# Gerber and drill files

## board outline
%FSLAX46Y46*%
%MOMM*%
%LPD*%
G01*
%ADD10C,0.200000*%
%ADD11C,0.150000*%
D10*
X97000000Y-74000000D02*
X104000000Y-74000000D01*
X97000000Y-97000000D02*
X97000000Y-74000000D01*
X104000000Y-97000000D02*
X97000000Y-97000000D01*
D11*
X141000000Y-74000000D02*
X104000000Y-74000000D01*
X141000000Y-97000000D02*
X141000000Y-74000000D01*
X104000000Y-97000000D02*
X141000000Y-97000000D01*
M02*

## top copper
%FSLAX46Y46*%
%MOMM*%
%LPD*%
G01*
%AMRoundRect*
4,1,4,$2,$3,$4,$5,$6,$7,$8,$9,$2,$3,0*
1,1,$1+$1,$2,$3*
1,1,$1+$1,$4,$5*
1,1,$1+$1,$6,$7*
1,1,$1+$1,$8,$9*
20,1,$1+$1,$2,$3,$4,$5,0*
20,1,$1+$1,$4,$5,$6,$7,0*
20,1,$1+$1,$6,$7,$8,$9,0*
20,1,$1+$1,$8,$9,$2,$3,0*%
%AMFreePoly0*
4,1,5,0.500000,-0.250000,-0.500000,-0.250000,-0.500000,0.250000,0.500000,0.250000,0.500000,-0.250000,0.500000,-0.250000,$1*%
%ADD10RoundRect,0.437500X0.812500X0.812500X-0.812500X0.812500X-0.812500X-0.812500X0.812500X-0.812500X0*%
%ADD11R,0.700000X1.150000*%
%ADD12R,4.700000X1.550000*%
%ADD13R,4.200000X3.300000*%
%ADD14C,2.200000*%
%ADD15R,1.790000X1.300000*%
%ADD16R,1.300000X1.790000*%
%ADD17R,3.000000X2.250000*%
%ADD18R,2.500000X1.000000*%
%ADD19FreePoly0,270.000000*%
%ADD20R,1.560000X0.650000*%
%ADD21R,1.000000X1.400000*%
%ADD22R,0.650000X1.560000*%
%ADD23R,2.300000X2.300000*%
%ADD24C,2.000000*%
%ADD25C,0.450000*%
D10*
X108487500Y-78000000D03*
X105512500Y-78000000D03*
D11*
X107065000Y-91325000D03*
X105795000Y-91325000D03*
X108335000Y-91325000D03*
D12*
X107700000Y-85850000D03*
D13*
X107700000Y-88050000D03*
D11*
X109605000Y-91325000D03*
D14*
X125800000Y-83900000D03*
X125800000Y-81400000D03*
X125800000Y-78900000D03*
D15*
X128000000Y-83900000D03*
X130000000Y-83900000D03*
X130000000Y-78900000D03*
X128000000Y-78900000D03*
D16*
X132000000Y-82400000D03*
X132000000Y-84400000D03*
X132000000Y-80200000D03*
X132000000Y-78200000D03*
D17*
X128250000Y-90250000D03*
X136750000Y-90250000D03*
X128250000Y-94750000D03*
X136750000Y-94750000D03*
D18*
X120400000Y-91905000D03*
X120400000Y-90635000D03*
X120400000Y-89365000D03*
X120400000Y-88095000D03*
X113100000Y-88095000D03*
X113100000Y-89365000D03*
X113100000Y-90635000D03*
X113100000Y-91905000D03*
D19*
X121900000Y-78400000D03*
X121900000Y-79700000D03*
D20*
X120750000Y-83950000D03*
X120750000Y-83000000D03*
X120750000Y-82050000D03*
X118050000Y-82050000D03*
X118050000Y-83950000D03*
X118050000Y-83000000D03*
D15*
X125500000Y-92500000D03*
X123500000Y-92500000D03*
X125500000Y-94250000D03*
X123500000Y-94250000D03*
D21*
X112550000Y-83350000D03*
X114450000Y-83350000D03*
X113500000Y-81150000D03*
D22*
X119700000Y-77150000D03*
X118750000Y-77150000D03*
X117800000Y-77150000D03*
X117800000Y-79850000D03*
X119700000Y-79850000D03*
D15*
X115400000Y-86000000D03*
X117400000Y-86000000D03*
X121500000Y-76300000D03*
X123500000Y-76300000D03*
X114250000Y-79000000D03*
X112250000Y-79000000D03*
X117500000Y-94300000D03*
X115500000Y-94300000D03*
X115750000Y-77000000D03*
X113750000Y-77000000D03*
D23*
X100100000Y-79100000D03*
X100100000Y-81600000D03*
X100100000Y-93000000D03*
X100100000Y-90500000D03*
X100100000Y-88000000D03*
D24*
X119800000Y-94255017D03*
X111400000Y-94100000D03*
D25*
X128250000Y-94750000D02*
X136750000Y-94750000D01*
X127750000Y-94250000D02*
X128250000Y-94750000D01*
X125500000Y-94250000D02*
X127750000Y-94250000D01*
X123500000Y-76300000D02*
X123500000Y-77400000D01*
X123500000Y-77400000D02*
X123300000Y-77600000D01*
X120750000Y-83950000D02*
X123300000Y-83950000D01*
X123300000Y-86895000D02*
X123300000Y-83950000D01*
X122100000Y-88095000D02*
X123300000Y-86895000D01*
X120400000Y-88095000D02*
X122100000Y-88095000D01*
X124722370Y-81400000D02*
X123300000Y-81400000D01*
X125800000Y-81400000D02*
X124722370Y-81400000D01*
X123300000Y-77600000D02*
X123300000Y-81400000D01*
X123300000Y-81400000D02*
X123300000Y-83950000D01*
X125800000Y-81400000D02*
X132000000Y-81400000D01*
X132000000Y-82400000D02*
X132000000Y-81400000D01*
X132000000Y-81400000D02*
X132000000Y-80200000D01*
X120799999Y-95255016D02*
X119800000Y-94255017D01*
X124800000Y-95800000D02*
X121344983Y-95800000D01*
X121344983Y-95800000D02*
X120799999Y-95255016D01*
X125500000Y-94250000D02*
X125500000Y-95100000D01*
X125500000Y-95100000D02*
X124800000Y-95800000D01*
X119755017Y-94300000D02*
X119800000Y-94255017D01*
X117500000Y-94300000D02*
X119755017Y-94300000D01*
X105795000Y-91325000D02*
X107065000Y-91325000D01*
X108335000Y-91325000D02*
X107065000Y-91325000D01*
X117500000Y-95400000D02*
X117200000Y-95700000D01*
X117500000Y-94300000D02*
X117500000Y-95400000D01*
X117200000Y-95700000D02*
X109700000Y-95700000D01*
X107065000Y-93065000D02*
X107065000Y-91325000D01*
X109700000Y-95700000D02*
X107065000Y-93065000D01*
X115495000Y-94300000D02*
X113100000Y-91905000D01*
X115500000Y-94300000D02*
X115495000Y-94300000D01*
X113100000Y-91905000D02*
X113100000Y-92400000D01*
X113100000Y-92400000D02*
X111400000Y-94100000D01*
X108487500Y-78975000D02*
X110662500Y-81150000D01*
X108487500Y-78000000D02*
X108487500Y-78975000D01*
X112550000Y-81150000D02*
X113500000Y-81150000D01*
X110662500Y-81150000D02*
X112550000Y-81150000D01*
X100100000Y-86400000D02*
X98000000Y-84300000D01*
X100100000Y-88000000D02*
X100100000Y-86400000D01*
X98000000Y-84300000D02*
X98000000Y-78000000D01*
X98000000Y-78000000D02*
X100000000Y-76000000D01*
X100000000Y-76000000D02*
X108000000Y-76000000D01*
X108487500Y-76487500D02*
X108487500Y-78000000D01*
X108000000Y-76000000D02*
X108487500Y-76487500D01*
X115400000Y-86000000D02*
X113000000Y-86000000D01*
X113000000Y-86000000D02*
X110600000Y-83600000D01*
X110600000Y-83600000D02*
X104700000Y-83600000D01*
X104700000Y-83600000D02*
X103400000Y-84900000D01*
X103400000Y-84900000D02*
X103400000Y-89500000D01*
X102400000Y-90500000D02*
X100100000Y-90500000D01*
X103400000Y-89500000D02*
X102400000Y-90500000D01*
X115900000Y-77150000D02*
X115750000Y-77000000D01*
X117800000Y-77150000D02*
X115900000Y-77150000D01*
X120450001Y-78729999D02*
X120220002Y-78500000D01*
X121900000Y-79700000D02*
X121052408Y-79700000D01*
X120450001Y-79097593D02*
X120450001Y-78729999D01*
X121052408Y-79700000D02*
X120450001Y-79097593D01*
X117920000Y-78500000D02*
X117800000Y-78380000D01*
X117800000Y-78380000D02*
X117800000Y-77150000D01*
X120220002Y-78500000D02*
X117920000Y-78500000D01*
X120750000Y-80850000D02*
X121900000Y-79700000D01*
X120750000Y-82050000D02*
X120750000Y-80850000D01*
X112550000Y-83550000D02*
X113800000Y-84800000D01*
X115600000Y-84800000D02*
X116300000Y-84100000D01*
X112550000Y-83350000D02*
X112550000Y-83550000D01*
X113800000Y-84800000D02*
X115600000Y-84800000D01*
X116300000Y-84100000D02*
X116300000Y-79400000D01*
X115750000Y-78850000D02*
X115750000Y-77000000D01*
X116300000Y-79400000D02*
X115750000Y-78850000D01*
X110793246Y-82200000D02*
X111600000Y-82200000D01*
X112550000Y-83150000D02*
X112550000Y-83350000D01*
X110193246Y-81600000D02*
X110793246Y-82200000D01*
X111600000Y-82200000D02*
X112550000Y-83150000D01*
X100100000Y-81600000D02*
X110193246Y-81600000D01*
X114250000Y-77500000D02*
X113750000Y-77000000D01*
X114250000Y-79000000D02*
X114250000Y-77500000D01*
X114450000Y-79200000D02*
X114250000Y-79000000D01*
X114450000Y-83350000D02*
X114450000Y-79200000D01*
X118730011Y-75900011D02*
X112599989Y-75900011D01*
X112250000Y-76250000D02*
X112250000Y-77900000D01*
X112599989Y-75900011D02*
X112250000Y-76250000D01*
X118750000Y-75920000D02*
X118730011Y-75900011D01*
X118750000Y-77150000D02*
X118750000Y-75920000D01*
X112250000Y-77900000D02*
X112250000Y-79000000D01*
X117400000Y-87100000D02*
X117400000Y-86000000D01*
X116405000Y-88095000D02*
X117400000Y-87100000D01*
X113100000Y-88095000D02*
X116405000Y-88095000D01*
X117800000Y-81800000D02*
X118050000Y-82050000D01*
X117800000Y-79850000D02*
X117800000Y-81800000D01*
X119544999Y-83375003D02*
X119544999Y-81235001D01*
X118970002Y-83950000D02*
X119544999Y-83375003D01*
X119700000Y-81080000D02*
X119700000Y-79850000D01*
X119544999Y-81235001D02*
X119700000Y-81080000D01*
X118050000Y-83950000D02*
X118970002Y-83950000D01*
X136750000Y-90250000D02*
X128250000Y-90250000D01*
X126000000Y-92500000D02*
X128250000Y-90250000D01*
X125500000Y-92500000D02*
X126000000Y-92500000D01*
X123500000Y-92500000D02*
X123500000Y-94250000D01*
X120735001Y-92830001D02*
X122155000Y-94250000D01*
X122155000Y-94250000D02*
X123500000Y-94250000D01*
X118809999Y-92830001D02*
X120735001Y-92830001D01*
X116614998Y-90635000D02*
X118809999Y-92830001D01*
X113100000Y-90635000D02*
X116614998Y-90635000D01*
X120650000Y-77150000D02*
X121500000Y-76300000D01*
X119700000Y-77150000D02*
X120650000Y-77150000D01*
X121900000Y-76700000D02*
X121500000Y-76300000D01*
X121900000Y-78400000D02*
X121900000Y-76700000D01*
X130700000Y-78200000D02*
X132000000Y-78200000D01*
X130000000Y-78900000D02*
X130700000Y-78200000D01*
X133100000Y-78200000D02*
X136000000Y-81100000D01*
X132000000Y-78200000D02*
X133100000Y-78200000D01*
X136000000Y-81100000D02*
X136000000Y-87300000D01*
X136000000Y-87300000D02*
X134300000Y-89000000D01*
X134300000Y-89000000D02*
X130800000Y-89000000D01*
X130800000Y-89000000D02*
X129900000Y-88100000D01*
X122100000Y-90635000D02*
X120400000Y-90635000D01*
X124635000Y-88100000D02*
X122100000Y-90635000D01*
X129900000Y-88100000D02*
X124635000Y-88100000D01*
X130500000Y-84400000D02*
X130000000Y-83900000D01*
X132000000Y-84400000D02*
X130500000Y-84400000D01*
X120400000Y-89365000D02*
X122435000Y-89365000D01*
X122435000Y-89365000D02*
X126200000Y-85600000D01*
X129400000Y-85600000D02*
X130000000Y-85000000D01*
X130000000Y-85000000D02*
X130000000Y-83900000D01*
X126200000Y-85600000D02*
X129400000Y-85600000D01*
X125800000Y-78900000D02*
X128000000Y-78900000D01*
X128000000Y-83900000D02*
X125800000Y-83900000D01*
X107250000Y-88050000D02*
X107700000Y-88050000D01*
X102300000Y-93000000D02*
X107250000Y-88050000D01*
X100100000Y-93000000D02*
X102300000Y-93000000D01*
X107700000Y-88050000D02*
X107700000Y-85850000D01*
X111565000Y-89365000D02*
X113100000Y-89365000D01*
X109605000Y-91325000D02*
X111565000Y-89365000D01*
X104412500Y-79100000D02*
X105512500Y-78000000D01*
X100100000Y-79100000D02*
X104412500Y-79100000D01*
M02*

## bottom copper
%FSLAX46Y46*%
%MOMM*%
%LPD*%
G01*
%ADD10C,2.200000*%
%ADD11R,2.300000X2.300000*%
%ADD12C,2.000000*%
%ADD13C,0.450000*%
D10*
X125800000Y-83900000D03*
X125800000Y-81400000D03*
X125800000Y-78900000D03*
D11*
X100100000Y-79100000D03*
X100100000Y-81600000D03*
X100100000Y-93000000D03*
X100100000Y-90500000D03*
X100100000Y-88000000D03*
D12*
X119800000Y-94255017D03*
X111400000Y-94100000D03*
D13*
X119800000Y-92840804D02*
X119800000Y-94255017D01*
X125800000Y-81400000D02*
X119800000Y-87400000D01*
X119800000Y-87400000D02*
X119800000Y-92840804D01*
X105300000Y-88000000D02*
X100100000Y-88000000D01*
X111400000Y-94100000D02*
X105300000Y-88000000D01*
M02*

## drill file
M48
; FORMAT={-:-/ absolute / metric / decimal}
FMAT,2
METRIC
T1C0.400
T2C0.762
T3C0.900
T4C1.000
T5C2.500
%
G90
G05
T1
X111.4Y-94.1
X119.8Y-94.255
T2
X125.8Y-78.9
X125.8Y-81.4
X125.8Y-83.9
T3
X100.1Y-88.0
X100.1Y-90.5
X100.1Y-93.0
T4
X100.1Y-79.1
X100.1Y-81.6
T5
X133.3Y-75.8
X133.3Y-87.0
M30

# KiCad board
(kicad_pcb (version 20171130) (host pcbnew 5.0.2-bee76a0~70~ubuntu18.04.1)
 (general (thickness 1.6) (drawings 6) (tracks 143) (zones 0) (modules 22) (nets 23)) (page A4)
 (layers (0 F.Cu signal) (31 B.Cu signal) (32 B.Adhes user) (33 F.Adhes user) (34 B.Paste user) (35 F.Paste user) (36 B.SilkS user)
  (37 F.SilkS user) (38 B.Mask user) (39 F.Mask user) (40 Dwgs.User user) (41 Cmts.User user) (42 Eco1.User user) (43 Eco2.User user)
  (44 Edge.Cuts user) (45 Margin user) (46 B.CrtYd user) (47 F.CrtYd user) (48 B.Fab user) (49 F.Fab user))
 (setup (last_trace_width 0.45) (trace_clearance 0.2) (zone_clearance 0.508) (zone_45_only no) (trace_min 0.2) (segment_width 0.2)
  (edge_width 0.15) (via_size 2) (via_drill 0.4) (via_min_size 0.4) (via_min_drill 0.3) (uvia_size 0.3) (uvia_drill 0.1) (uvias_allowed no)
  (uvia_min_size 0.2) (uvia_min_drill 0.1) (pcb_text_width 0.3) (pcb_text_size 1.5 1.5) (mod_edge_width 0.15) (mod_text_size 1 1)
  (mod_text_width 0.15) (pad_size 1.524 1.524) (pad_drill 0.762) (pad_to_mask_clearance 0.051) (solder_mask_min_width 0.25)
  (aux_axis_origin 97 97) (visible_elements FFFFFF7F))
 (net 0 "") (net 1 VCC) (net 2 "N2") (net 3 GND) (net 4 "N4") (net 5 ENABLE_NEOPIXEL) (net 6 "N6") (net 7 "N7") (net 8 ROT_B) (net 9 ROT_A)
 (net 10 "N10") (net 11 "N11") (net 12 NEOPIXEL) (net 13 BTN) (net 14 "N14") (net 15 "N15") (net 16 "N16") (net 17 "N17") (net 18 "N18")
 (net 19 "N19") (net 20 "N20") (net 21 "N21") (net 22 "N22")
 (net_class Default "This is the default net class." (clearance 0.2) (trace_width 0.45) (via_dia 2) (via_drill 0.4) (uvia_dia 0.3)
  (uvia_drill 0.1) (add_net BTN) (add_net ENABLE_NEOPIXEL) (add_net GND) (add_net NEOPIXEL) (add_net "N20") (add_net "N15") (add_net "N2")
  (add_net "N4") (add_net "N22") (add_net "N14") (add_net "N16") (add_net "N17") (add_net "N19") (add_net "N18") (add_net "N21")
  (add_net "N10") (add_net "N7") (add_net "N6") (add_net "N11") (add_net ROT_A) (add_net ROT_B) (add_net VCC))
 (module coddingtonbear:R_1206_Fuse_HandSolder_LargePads (layer F.Cu) (at 107 78 180)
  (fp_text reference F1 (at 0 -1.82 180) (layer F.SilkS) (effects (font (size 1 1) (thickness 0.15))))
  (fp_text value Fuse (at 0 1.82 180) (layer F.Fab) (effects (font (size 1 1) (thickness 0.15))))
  (pad 1 smd roundrect (at -1.4875 0 180) (size 2.5 2.5) (layers F.Cu F.Paste F.Mask) (roundrect_rratio 0.175) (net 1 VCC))
  (pad 2 smd roundrect (at 1.4875 0 180) (size 2.5 2.5) (layers F.Cu F.Paste F.Mask) (roundrect_rratio 0.175) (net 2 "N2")))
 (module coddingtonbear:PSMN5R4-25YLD (layer F.Cu) (at 107.7 88.5)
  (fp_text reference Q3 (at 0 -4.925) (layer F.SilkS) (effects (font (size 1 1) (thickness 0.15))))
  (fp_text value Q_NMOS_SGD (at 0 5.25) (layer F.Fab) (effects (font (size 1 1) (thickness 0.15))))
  (pad 7 smd rect (at -1.15 -0.2 90) (size 0.6 0.9) (layers F.Paste))
  (pad 7 smd rect (at -1.15 0.65 90) (size 0.6 0.9) (layers F.Paste))
  (pad 7 smd rect (at -1.15 -1.05 90) (size 0.6 0.9) (layers F.Paste))
  (pad 7 smd rect (at 1.15 -0.2 90) (size 0.6 0.9) (layers F.Paste))
  (pad 7 smd rect (at 1.15 0.65 90) (size 0.6 0.9) (layers F.Paste))
  (pad 7 smd rect (at 1.15 -1.05 90) (size 0.6 0.9) (layers F.Paste))
  (pad 7 smd rect (at 0 -1.05 90) (size 0.6 0.9) (layers F.Paste))
  (pad 7 smd rect (at 0 0.65 90) (size 0.6 0.9) (layers F.Paste))
  (pad 6 smd rect (at -1.875 -2.9) (size 0.6 0.9) (layers F.Paste))
  (pad 6 smd rect (at 1.875 -2.9) (size 0.6 0.9) (layers F.Paste))
  (pad 6 smd rect (at -0.6 -2.9) (size 0.6 0.9) (layers F.Paste))
  (pad 1 smd rect (at -0.635 2.825) (size 0.7 1.15) (layers F.Cu F.Paste F.Mask) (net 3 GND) (solder_mask_margin 0.075)
   (solder_paste_margin -0.05))
  (pad 1 smd rect (at -1.905 2.825) (size 0.7 1.15) (layers F.Cu F.Paste F.Mask) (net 3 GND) (solder_mask_margin 0.075)
   (solder_paste_margin -0.05))
  (pad 1 smd rect (at 0.635 2.825) (size 0.7 1.15) (layers F.Cu F.Paste F.Mask) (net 3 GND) (solder_mask_margin 0.075)
   (solder_paste_margin -0.05))
  (pad 3 smd rect (at 0 -2.65) (size 4.7 1.55) (layers F.Cu F.Mask) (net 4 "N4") (solder_mask_margin 0.075))
  (pad 3 smd rect (at 0 -0.45) (size 4.2 3.3) (layers F.Cu F.Mask) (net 4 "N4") (solder_mask_margin 0.075))
  (pad 2 smd rect (at 1.905 2.825) (size 0.7 1.15) (layers F.Cu F.Paste F.Mask) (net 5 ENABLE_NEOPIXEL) (solder_mask_margin 0.075)
   (solder_paste_margin -0.05))
  (pad 6 smd rect (at 0.6 -2.9) (size 0.6 0.9) (layers F.Paste))
  (pad 7 smd rect (at 0 -0.2 90) (size 0.6 0.9) (layers F.Paste)))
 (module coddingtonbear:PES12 (layer F.Cu) (at 133.3 81.4 270)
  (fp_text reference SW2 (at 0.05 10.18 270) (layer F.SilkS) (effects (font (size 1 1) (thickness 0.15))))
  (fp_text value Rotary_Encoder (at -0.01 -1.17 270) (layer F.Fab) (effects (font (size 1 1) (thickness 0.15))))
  (pad "" np_thru_hole circle (at 5.6 0 270) (size 2.5 2.5) (drill 2.5) (layers *.Cu *.Mask))
  (pad "" np_thru_hole circle (at -5.6 0 270) (size 2.5 2.5) (drill 2.5) (layers *.Cu *.Mask))
  (pad B thru_hole circle (at 2.5 7.5 270) (size 2.2 2.2) (drill 0.762) (layers *.Cu *.Mask) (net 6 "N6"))
  (pad C thru_hole circle (at 0 7.5 270) (size 2.2 2.2) (drill 0.762) (layers *.Cu *.Mask) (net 3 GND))
  (pad A thru_hole circle (at -2.5 7.5 270) (size 2.2 2.2) (drill 0.762) (layers *.Cu *.Mask) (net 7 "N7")))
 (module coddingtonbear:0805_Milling (layer F.Cu) (at 129 83.9)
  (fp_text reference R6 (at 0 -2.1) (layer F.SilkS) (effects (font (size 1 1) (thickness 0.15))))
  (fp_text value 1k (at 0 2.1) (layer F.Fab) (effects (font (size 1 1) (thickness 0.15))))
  (pad 1 smd rect (at -1 0) (size 1.79 1.3) (layers F.Cu F.Paste F.Mask) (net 6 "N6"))
  (pad 2 smd rect (at 1 0) (size 1.79 1.3) (layers F.Cu F.Paste F.Mask) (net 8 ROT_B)))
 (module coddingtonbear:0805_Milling (layer F.Cu) (at 129 78.9)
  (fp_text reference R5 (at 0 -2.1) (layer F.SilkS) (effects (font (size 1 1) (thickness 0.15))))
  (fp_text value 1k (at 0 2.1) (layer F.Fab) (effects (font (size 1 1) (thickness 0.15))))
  (pad 2 smd rect (at 1 0) (size 1.79 1.3) (layers F.Cu F.Paste F.Mask) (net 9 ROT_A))
  (pad 1 smd rect (at -1 0) (size 1.79 1.3) (layers F.Cu F.Paste F.Mask) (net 7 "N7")))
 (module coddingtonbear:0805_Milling (layer F.Cu) (at 132 83.4 270)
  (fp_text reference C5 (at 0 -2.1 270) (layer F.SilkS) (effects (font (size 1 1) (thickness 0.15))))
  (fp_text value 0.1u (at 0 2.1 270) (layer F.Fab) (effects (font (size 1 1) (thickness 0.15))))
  (pad 1 smd rect (at -1 0 270) (size 1.79 1.3) (layers F.Cu F.Paste F.Mask) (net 3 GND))
  (pad 2 smd rect (at 1 0 270) (size 1.79 1.3) (layers F.Cu F.Paste F.Mask) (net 8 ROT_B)))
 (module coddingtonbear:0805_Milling (layer F.Cu) (at 132 79.2 270)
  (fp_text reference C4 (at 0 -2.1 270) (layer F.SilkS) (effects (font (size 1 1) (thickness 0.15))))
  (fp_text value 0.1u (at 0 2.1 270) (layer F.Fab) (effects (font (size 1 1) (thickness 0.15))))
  (pad 2 smd rect (at 1 0 270) (size 1.79 1.3) (layers F.Cu F.Paste F.Mask) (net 3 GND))
  (pad 1 smd rect (at -1 0 270) (size 1.79 1.3) (layers F.Cu F.Paste F.Mask) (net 9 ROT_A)))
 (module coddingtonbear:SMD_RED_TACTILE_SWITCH (layer F.Cu) (at 132.5 92.5)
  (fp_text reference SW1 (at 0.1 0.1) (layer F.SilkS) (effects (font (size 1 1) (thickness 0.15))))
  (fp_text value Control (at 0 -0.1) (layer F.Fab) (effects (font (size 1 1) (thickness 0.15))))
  (pad 1 smd rect (at -4.25 -2.25) (size 3 2.25) (layers F.Cu F.Paste F.Mask) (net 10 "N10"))
  (pad 1 smd rect (at 4.25 -2.25) (size 3 2.25) (layers F.Cu F.Paste F.Mask) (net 10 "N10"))
  (pad 2 smd rect (at -4.25 2.25) (size 3 2.25) (layers F.Cu F.Paste F.Mask) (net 3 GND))
  (pad 2 smd rect (at 4.25 2.25) (size 3 2.25) (layers F.Cu F.Paste F.Mask) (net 3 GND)))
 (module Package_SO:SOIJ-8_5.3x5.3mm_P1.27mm (layer F.Cu) (at 116.75 90 180)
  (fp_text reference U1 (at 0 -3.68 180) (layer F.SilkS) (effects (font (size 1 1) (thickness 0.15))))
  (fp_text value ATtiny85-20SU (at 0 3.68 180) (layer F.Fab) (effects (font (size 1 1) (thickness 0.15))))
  (pad 1 smd rect (at -3.65 -1.905 180) (size 2.5 1) (layers F.Cu F.Paste F.Mask) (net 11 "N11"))
  (pad 2 smd rect (at -3.65 -0.635 180) (size 2.5 1) (layers F.Cu F.Paste F.Mask) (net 9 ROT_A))
  (pad 3 smd rect (at -3.65 0.635 180) (size 2.5 1) (layers F.Cu F.Paste F.Mask) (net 8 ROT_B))
  (pad 4 smd rect (at -3.65 1.905 180) (size 2.5 1) (layers F.Cu F.Paste F.Mask) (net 3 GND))
  (pad 5 smd rect (at 3.65 1.905 180) (size 2.5 1) (layers F.Cu F.Paste F.Mask) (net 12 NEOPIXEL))
  (pad 6 smd rect (at 3.65 0.635 180) (size 2.5 1) (layers F.Cu F.Paste F.Mask) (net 5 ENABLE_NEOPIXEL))
  (pad 7 smd rect (at 3.65 -0.635 180) (size 2.5 1) (layers F.Cu F.Paste F.Mask) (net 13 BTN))
  (pad 8 smd rect (at 3.65 -1.905 180) (size 2.5 1) (layers F.Cu F.Paste F.Mask) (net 1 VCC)))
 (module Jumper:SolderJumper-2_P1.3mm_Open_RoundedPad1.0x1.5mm (layer F.Cu) (at 121.9 79.05 270)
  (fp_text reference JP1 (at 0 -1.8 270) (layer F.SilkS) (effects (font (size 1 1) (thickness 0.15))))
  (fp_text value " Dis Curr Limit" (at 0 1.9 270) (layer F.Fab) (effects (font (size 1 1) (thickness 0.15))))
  (pad 1 smd custom (at -0.65 0 270) (size 1 0.5) (layers F.Cu F.Mask) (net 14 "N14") (zone_connect 0)
   (options (clearance outline) (anchor rect)) (primitives))
  (pad 2 smd custom (at 0.65 0 270) (size 1 0.5) (layers F.Cu F.Mask) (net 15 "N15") (zone_connect 0)
   (options (clearance outline) (anchor rect)) (primitives)))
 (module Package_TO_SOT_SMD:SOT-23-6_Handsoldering (layer F.Cu) (at 119.4 83 180)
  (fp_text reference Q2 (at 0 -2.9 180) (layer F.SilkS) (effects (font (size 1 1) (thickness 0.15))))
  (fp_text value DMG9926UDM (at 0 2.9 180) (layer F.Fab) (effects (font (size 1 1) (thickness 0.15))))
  (pad 1 smd rect (at -1.35 -0.95 180) (size 1.56 0.65) (layers F.Cu F.Paste F.Mask) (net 3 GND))
  (pad 2 smd rect (at -1.35 0 180) (size 1.56 0.65) (layers F.Cu F.Paste F.Mask) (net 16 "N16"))
  (pad 3 smd rect (at -1.35 0.95 180) (size 1.56 0.65) (layers F.Cu F.Paste F.Mask) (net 15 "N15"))
  (pad 4 smd rect (at 1.35 0.95 180) (size 1.56 0.65) (layers F.Cu F.Paste F.Mask) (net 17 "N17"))
  (pad 6 smd rect (at 1.35 -0.95 180) (size 1.56 0.65) (layers F.Cu F.Paste F.Mask) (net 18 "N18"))
  (pad 5 smd rect (at 1.35 0 180) (size 1.56 0.65) (layers F.Cu F.Paste F.Mask) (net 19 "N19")))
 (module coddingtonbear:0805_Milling (layer F.Cu) (at 124.5 92.5 180)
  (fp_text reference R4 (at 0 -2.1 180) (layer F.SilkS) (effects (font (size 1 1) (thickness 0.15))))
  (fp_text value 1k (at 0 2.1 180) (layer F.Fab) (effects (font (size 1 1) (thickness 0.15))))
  (pad 1 smd rect (at -1 0 180) (size 1.79 1.3) (layers F.Cu F.Paste F.Mask) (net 10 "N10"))
  (pad 2 smd rect (at 1 0 180) (size 1.79 1.3) (layers F.Cu F.Paste F.Mask) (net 13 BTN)))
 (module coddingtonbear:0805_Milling (layer F.Cu) (at 124.5 94.25)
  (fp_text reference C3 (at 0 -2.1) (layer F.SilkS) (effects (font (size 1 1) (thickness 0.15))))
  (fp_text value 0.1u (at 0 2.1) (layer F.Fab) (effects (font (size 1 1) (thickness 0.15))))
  (pad 2 smd rect (at 1 0) (size 1.79 1.3) (layers F.Cu F.Paste F.Mask) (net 3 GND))
  (pad 1 smd rect (at -1 0) (size 1.79 1.3) (layers F.Cu F.Paste F.Mask) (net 13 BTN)))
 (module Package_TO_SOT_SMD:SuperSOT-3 (layer F.Cu) (at 113.5 82.25 90)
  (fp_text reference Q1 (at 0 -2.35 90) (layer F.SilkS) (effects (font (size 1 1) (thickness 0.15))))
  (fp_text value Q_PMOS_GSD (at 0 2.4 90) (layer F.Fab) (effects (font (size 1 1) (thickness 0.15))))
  (pad 1 smd rect (at -1.1 -0.95 90) (size 1.4 1) (layers F.Cu F.Paste F.Mask) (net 15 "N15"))
  (pad 2 smd rect (at -1.1 0.95 90) (size 1.4 1) (layers F.Cu F.Paste F.Mask) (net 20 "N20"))
  (pad 3 smd rect (at 1.1 0 90) (size 1.4 1) (layers F.Cu F.Paste F.Mask) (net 1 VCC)))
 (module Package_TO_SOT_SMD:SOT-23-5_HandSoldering (layer F.Cu) (at 118.75 78.5 270)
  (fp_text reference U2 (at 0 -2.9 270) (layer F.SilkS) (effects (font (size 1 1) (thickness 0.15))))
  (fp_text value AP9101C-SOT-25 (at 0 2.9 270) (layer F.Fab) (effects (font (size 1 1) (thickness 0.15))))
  (pad 1 smd rect (at -1.35 -0.95 270) (size 1.56 0.65) (layers F.Cu F.Paste F.Mask) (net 14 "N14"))
  (pad 2 smd rect (at -1.35 0 270) (size 1.56 0.65) (layers F.Cu F.Paste F.Mask) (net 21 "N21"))
  (pad 3 smd rect (at -1.35 0.95 270) (size 1.56 0.65) (layers F.Cu F.Paste F.Mask) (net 15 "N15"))
  (pad 4 smd rect (at 1.35 0.95 270) (size 1.56 0.65) (layers F.Cu F.Paste F.Mask) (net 17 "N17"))
  (pad 5 smd rect (at 1.35 -0.95 270) (size 1.56 0.65) (layers F.Cu F.Paste F.Mask) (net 18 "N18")))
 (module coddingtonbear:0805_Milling (layer F.Cu) (at 116.4 86 180)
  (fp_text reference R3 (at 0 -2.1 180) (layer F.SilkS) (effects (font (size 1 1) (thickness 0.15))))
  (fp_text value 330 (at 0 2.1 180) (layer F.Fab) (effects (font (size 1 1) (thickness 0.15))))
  (pad 2 smd rect (at 1 0 180) (size 1.79 1.3) (layers F.Cu F.Paste F.Mask) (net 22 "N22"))
  (pad 1 smd rect (at -1 0 180) (size 1.79 1.3) (layers F.Cu F.Paste F.Mask) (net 12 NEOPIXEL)))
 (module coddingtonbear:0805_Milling (layer F.Cu) (at 122.5 76.3)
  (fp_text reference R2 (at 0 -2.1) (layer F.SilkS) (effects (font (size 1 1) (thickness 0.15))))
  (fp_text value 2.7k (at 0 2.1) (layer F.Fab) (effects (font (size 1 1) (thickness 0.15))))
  (pad 1 smd rect (at -1 0) (size 1.79 1.3) (layers F.Cu F.Paste F.Mask) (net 14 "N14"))
  (pad 2 smd rect (at 1 0) (size 1.79 1.3) (layers F.Cu F.Paste F.Mask) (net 3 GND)))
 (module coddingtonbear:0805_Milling (layer F.Cu) (at 113.25 79)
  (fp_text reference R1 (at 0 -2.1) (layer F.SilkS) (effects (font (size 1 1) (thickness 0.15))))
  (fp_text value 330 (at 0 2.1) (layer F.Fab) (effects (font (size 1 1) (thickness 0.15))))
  (pad 2 smd rect (at 1 0) (size 1.79 1.3) (layers F.Cu F.Paste F.Mask) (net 20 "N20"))
  (pad 1 smd rect (at -1 0) (size 1.79 1.3) (layers F.Cu F.Paste F.Mask) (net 21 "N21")))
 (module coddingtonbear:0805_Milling (layer F.Cu) (at 116.5 94.3 180)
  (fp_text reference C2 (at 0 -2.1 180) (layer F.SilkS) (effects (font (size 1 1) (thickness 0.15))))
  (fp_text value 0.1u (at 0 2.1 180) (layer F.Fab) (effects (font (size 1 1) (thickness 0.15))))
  (pad 1 smd rect (at -1 0 180) (size 1.79 1.3) (layers F.Cu F.Paste F.Mask) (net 3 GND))
  (pad 2 smd rect (at 1 0 180) (size 1.79 1.3) (layers F.Cu F.Paste F.Mask) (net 1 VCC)))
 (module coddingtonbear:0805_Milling (layer F.Cu) (at 114.75 77)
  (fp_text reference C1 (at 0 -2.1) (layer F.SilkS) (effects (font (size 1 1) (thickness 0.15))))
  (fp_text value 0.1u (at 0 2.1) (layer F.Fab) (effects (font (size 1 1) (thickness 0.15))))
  (pad 2 smd rect (at 1 0) (size 1.79 1.3) (layers F.Cu F.Paste F.Mask) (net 15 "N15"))
  (pad 1 smd rect (at -1 0) (size 1.79 1.3) (layers F.Cu F.Paste F.Mask) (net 20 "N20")))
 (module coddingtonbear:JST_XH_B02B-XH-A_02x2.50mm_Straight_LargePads (layer F.Cu) (at 100.1 81.6 90)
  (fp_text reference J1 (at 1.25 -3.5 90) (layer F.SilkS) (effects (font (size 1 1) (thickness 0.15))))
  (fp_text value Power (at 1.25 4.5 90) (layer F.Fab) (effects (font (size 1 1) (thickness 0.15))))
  (pad 2 thru_hole rect (at 2.5 0 90) (size 2.3 2.3) (drill 1) (layers *.Cu *.Mask) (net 2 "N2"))
  (pad 1 thru_hole rect (at 0 0 90) (size 2.3 2.3) (drill 1) (layers *.Cu *.Mask) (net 15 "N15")))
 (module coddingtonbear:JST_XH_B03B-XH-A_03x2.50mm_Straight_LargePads (layer F.Cu) (at 100.1 93 90)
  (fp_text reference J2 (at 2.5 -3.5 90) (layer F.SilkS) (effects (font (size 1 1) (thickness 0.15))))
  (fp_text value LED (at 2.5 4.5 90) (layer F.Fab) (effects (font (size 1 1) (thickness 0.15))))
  (pad 1 thru_hole rect (at 0 0 90) (size 2.3 2.3) (drill 0.9) (layers *.Cu *.Mask) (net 4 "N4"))
  (pad 2 thru_hole rect (at 2.5 0 90) (size 2.3 2.3) (drill 0.9) (layers *.Cu *.Mask) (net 22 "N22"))
  (pad 3 thru_hole rect (at 5 0 90) (size 2.3 2.3) (drill 0.9) (layers *.Cu *.Mask) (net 1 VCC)))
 (gr_line (start 97 74) (end 104 74) (layer Edge.Cuts) (width 0.2))
 (gr_line (start 97 97) (end 97 74) (layer Edge.Cuts) (width 0.2))
 (gr_line (start 104 97) (end 97 97) (layer Edge.Cuts) (width 0.2))
 (gr_line (start 141 74) (end 104 74) (layer Edge.Cuts) (width 0.15))
 (gr_line (start 141 97) (end 141 74) (layer Edge.Cuts) (width 0.15))
 (gr_line (start 104 97) (end 141 97) (layer Edge.Cuts) (width 0.15))
 (segment (start 128.25 94.75) (end 136.75 94.75) (width 0.45) (layer F.Cu) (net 3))
 (segment (start 127.75 94.25) (end 128.25 94.75) (width 0.45) (layer F.Cu) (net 3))
 (segment (start 125.5 94.25) (end 127.75 94.25) (width 0.45) (layer F.Cu) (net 3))
 (segment (start 123.5 76.3) (end 123.5 77.4) (width 0.45) (layer F.Cu) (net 3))
 (segment (start 123.5 77.4) (end 123.3 77.6) (width 0.45) (layer F.Cu) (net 3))
 (segment (start 120.75 83.95) (end 123.3 83.95) (width 0.45) (layer F.Cu) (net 3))
 (segment (start 123.3 86.895) (end 123.3 83.95) (width 0.45) (layer F.Cu) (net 3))
 (segment (start 122.1 88.095) (end 123.3 86.895) (width 0.45) (layer F.Cu) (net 3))
 (segment (start 120.4 88.095) (end 122.1 88.095) (width 0.45) (layer F.Cu) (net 3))
 (segment (start 124.72237 81.4) (end 123.3 81.4) (width 0.45) (layer F.Cu) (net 3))
 (segment (start 125.8 81.4) (end 124.72237 81.4) (width 0.45) (layer F.Cu) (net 3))
 (segment (start 123.3 77.6) (end 123.3 81.4) (width 0.45) (layer F.Cu) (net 3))
 (segment (start 123.3 81.4) (end 123.3 83.95) (width 0.45) (layer F.Cu) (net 3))
 (segment (start 125.8 81.4) (end 132 81.4) (width 0.45) (layer F.Cu) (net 3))
 (segment (start 132 82.4) (end 132 81.4) (width 0.45) (layer F.Cu) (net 3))
 (segment (start 132 81.4) (end 132 80.2) (width 0.45) (layer F.Cu) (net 3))
 (via (at 119.8 94.255017) (size 2) (drill 0.4) (layers F.Cu B.Cu) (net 3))
 (segment (start 119.8 92.840804) (end 119.8 94.255017) (width 0.45) (layer B.Cu) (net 3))
 (segment (start 125.8 81.4) (end 119.8 87.4) (width 0.45) (layer B.Cu) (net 3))
 (segment (start 119.8 87.4) (end 119.8 92.840804) (width 0.45) (layer B.Cu) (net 3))
 (segment (start 120.799999 95.255016) (end 119.8 94.255017) (width 0.45) (layer F.Cu) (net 3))
 (segment (start 124.8 95.8) (end 121.344983 95.8) (width 0.45) (layer F.Cu) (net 3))
 (segment (start 121.344983 95.8) (end 120.799999 95.255016) (width 0.45) (layer F.Cu) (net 3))
 (segment (start 125.5 94.25) (end 125.5 95.1) (width 0.45) (layer F.Cu) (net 3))
 (segment (start 125.5 95.1) (end 124.8 95.8) (width 0.45) (layer F.Cu) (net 3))
 (segment (start 119.755017 94.3) (end 119.8 94.255017) (width 0.45) (layer F.Cu) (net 3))
 (segment (start 117.5 94.3) (end 119.755017 94.3) (width 0.45) (layer F.Cu) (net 3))
 (segment (start 105.795 91.325) (end 107.065 91.325) (width 0.45) (layer F.Cu) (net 3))
 (segment (start 108.335 91.325) (end 107.065 91.325) (width 0.45) (layer F.Cu) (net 3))
 (segment (start 117.5 95.4) (end 117.2 95.7) (width 0.45) (layer F.Cu) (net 3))
 (segment (start 117.5 94.3) (end 117.5 95.4) (width 0.45) (layer F.Cu) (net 3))
 (segment (start 117.2 95.7) (end 109.7 95.7) (width 0.45) (layer F.Cu) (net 3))
 (segment (start 107.065 93.065) (end 107.065 91.325) (width 0.45) (layer F.Cu) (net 3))
 (segment (start 109.7 95.7) (end 107.065 93.065) (width 0.45) (layer F.Cu) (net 3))
 (segment (start 115.495 94.3) (end 113.1 91.905) (width 0.45) (layer F.Cu) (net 1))
 (segment (start 115.5 94.3) (end 115.495 94.3) (width 0.45) (layer F.Cu) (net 1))
 (via (at 111.4 94.1) (size 2) (drill 0.4) (layers F.Cu B.Cu) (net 1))
 (segment (start 113.1 91.905) (end 113.1 92.4) (width 0.45) (layer F.Cu) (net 1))
 (segment (start 113.1 92.4) (end 111.4 94.1) (width 0.45) (layer F.Cu) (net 1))
 (segment (start 105.3 88) (end 100.1 88) (width 0.45) (layer B.Cu) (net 1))
 (segment (start 111.4 94.1) (end 105.3 88) (width 0.45) (layer B.Cu) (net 1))
 (segment (start 108.4875 78.975) (end 110.6625 81.15) (width 0.45) (layer F.Cu) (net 1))
 (segment (start 108.4875 78) (end 108.4875 78.975) (width 0.45) (layer F.Cu) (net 1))
 (segment (start 112.55 81.15) (end 113.5 81.15) (width 0.45) (layer F.Cu) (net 1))
 (segment (start 110.6625 81.15) (end 112.55 81.15) (width 0.45) (layer F.Cu) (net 1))
 (segment (start 100.1 86.4) (end 98 84.3) (width 0.45) (layer F.Cu) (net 1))
 (segment (start 100.1 88) (end 100.1 86.4) (width 0.45) (layer F.Cu) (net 1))
 (segment (start 98 84.3) (end 98 78) (width 0.45) (layer F.Cu) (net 1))
 (segment (start 98 78) (end 100 76) (width 0.45) (layer F.Cu) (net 1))
 (segment (start 100 76) (end 108 76) (width 0.45) (layer F.Cu) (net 1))
 (segment (start 108.4875 76.4875) (end 108.4875 78) (width 0.45) (layer F.Cu) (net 1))
 (segment (start 108 76) (end 108.4875 76.4875) (width 0.45) (layer F.Cu) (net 1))
 (segment (start 115.4 86) (end 113 86) (width 0.45) (layer F.Cu) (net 22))
 (segment (start 113 86) (end 110.6 83.6) (width 0.45) (layer F.Cu) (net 22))
 (segment (start 110.6 83.6) (end 104.7 83.6) (width 0.45) (layer F.Cu) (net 22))
 (segment (start 104.7 83.6) (end 103.4 84.9) (width 0.45) (layer F.Cu) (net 22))
 (segment (start 103.4 84.9) (end 103.4 89.5) (width 0.45) (layer F.Cu) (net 22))
 (segment (start 102.4 90.5) (end 100.1 90.5) (width 0.45) (layer F.Cu) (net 22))
 (segment (start 103.4 89.5) (end 102.4 90.5) (width 0.45) (layer F.Cu) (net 22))
 (segment (start 115.9 77.15) (end 115.75 77) (width 0.45) (layer F.Cu) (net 15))
 (segment (start 117.8 77.15) (end 115.9 77.15) (width 0.45) (layer F.Cu) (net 15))
 (segment (start 120.450001 78.729999) (end 120.220002 78.5) (width 0.45) (layer F.Cu) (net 15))
 (segment (start 121.9 79.7) (end 121.052408 79.7) (width 0.45) (layer F.Cu) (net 15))
 (segment (start 120.450001 79.097593) (end 120.450001 78.729999) (width 0.45) (layer F.Cu) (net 15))
 (segment (start 121.052408 79.7) (end 120.450001 79.097593) (width 0.45) (layer F.Cu) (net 15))
 (segment (start 117.92 78.5) (end 117.8 78.38) (width 0.45) (layer F.Cu) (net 15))
 (segment (start 117.8 78.38) (end 117.8 77.15) (width 0.45) (layer F.Cu) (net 15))
 (segment (start 120.220002 78.5) (end 117.92 78.5) (width 0.45) (layer F.Cu) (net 15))
 (segment (start 120.75 80.85) (end 121.9 79.7) (width 0.45) (layer F.Cu) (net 15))
 (segment (start 120.75 82.05) (end 120.75 80.85) (width 0.45) (layer F.Cu) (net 15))
 (segment (start 112.55 83.55) (end 113.8 84.8) (width 0.45) (layer F.Cu) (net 15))
 (segment (start 115.6 84.8) (end 116.3 84.1) (width 0.45) (layer F.Cu) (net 15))
 (segment (start 112.55 83.35) (end 112.55 83.55) (width 0.45) (layer F.Cu) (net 15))
 (segment (start 113.8 84.8) (end 115.6 84.8) (width 0.45) (layer F.Cu) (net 15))
 (segment (start 116.3 84.1) (end 116.3 79.4) (width 0.45) (layer F.Cu) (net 15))
 (segment (start 115.75 78.85) (end 115.75 77) (width 0.45) (layer F.Cu) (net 15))
 (segment (start 116.3 79.4) (end 115.75 78.85) (width 0.45) (layer F.Cu) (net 15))
 (segment (start 110.793246 82.2) (end 111.6 82.2) (width 0.45) (layer F.Cu) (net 15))
 (segment (start 112.55 83.15) (end 112.55 83.35) (width 0.45) (layer F.Cu) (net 15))
 (segment (start 110.193246 81.6) (end 110.793246 82.2) (width 0.45) (layer F.Cu) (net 15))
 (segment (start 111.6 82.2) (end 112.55 83.15) (width 0.45) (layer F.Cu) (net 15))
 (segment (start 100.1 81.6) (end 110.193246 81.6) (width 0.45) (layer F.Cu) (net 15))
 (segment (start 114.25 77.5) (end 113.75 77) (width 0.45) (layer F.Cu) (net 20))
 (segment (start 114.25 79) (end 114.25 77.5) (width 0.45) (layer F.Cu) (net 20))
 (segment (start 114.45 79.2) (end 114.25 79) (width 0.45) (layer F.Cu) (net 20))
 (segment (start 114.45 83.35) (end 114.45 79.2) (width 0.45) (layer F.Cu) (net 20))
 (segment (start 118.730011 75.900011) (end 112.599989 75.900011) (width 0.45) (layer F.Cu) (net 21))
 (segment (start 112.25 76.25) (end 112.25 77.9) (width 0.45) (layer F.Cu) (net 21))
 (segment (start 112.599989 75.900011) (end 112.25 76.25) (width 0.45) (layer F.Cu) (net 21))
 (segment (start 118.75 75.92) (end 118.730011 75.900011) (width 0.45) (layer F.Cu) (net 21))
 (segment (start 118.75 77.15) (end 118.75 75.92) (width 0.45) (layer F.Cu) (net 21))
 (segment (start 112.25 77.9) (end 112.25 79) (width 0.45) (layer F.Cu) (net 21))
 (segment (start 117.4 87.1) (end 117.4 86) (width 0.45) (layer F.Cu) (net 12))
 (segment (start 116.405 88.095) (end 117.4 87.1) (width 0.45) (layer F.Cu) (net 12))
 (segment (start 113.1 88.095) (end 116.405 88.095) (width 0.45) (layer F.Cu) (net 12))
 (segment (start 117.8 81.8) (end 118.05 82.05) (width 0.45) (layer F.Cu) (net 17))
 (segment (start 117.8 79.85) (end 117.8 81.8) (width 0.45) (layer F.Cu) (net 17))
 (segment (start 119.544999 83.375003) (end 119.544999 81.235001) (width 0.45) (layer F.Cu) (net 18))
 (segment (start 118.970002 83.95) (end 119.544999 83.375003) (width 0.45) (layer F.Cu) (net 18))
 (segment (start 119.7 81.08) (end 119.7 79.85) (width 0.45) (layer F.Cu) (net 18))
 (segment (start 119.544999 81.235001) (end 119.7 81.08) (width 0.45) (layer F.Cu) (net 18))
 (segment (start 118.05 83.95) (end 118.970002 83.95) (width 0.45) (layer F.Cu) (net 18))
 (segment (start 136.75 90.25) (end 128.25 90.25) (width 0.45) (layer F.Cu) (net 10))
 (segment (start 126 92.5) (end 128.25 90.25) (width 0.45) (layer F.Cu) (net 10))
 (segment (start 125.5 92.5) (end 126 92.5) (width 0.45) (layer F.Cu) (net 10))
 (segment (start 123.5 92.5) (end 123.5 94.25) (width 0.45) (layer F.Cu) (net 13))
 (segment (start 120.735001 92.830001) (end 122.155 94.25) (width 0.45) (layer F.Cu) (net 13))
 (segment (start 122.155 94.25) (end 123.5 94.25) (width 0.45) (layer F.Cu) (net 13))
 (segment (start 118.809999 92.830001) (end 120.735001 92.830001) (width 0.45) (layer F.Cu) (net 13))
 (segment (start 116.614998 90.635) (end 118.809999 92.830001) (width 0.45) (layer F.Cu) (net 13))
 (segment (start 113.1 90.635) (end 116.614998 90.635) (width 0.45) (layer F.Cu) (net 13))
 (segment (start 120.65 77.15) (end 121.5 76.3) (width 0.45) (layer F.Cu) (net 14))
 (segment (start 119.7 77.15) (end 120.65 77.15) (width 0.45) (layer F.Cu) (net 14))
 (segment (start 121.9 76.7) (end 121.5 76.3) (width 0.45) (layer F.Cu) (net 14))
 (segment (start 121.9 78.4) (end 121.9 76.7) (width 0.45) (layer F.Cu) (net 14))
 (segment (start 130.7 78.2) (end 132 78.2) (width 0.45) (layer F.Cu) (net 9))
 (segment (start 130 78.9) (end 130.7 78.2) (width 0.45) (layer F.Cu) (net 9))
 (segment (start 133.1 78.2) (end 136 81.1) (width 0.45) (layer F.Cu) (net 9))
 (segment (start 132 78.2) (end 133.1 78.2) (width 0.45) (layer F.Cu) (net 9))
 (segment (start 136 81.1) (end 136 87.3) (width 0.45) (layer F.Cu) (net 9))
 (segment (start 136 87.3) (end 134.3 89) (width 0.45) (layer F.Cu) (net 9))
 (segment (start 134.3 89) (end 130.8 89) (width 0.45) (layer F.Cu) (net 9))
 (segment (start 130.8 89) (end 129.9 88.1) (width 0.45) (layer F.Cu) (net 9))
 (segment (start 122.1 90.635) (end 120.4 90.635) (width 0.45) (layer F.Cu) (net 9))
 (segment (start 124.635 88.1) (end 122.1 90.635) (width 0.45) (layer F.Cu) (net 9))
 (segment (start 129.9 88.1) (end 124.635 88.1) (width 0.45) (layer F.Cu) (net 9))
 (segment (start 130.5 84.4) (end 130 83.9) (width 0.45) (layer F.Cu) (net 8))
 (segment (start 132 84.4) (end 130.5 84.4) (width 0.45) (layer F.Cu) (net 8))
 (segment (start 120.4 89.365) (end 122.435 89.365) (width 0.45) (layer F.Cu) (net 8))
 (segment (start 122.435 89.365) (end 126.2 85.6) (width 0.45) (layer F.Cu) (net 8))
 (segment (start 129.4 85.6) (end 130 85) (width 0.45) (layer F.Cu) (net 8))
 (segment (start 130 85) (end 130 83.9) (width 0.45) (layer F.Cu) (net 8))
 (segment (start 126.2 85.6) (end 129.4 85.6) (width 0.45) (layer F.Cu) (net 8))
 (segment (start 125.8 78.9) (end 128 78.9) (width 0.45) (layer F.Cu) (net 7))
 (segment (start 128 83.9) (end 125.8 83.9) (width 0.45) (layer F.Cu) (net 6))
 (segment (start 107.25 88.05) (end 107.7 88.05) (width 0.45) (layer F.Cu) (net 4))
 (segment (start 102.3 93) (end 107.25 88.05) (width 0.45) (layer F.Cu) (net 4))
 (segment (start 100.1 93) (end 102.3 93) (width 0.45) (layer F.Cu) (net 4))
 (segment (start 107.7 88.05) (end 107.7 85.85) (width 0.45) (layer F.Cu) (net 4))
 (segment (start 111.565 89.365) (end 113.1 89.365) (width 0.45) (layer F.Cu) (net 5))
 (segment (start 109.605 91.325) (end 111.565 89.365) (width 0.45) (layer F.Cu) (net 5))
 (segment (start 104.4125 79.1) (end 105.5125 78) (width 0.45) (layer F.Cu) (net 2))
 (segment (start 100.1 79.1) (end 104.4125 79.1) (width 0.45) (layer F.Cu) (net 2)))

